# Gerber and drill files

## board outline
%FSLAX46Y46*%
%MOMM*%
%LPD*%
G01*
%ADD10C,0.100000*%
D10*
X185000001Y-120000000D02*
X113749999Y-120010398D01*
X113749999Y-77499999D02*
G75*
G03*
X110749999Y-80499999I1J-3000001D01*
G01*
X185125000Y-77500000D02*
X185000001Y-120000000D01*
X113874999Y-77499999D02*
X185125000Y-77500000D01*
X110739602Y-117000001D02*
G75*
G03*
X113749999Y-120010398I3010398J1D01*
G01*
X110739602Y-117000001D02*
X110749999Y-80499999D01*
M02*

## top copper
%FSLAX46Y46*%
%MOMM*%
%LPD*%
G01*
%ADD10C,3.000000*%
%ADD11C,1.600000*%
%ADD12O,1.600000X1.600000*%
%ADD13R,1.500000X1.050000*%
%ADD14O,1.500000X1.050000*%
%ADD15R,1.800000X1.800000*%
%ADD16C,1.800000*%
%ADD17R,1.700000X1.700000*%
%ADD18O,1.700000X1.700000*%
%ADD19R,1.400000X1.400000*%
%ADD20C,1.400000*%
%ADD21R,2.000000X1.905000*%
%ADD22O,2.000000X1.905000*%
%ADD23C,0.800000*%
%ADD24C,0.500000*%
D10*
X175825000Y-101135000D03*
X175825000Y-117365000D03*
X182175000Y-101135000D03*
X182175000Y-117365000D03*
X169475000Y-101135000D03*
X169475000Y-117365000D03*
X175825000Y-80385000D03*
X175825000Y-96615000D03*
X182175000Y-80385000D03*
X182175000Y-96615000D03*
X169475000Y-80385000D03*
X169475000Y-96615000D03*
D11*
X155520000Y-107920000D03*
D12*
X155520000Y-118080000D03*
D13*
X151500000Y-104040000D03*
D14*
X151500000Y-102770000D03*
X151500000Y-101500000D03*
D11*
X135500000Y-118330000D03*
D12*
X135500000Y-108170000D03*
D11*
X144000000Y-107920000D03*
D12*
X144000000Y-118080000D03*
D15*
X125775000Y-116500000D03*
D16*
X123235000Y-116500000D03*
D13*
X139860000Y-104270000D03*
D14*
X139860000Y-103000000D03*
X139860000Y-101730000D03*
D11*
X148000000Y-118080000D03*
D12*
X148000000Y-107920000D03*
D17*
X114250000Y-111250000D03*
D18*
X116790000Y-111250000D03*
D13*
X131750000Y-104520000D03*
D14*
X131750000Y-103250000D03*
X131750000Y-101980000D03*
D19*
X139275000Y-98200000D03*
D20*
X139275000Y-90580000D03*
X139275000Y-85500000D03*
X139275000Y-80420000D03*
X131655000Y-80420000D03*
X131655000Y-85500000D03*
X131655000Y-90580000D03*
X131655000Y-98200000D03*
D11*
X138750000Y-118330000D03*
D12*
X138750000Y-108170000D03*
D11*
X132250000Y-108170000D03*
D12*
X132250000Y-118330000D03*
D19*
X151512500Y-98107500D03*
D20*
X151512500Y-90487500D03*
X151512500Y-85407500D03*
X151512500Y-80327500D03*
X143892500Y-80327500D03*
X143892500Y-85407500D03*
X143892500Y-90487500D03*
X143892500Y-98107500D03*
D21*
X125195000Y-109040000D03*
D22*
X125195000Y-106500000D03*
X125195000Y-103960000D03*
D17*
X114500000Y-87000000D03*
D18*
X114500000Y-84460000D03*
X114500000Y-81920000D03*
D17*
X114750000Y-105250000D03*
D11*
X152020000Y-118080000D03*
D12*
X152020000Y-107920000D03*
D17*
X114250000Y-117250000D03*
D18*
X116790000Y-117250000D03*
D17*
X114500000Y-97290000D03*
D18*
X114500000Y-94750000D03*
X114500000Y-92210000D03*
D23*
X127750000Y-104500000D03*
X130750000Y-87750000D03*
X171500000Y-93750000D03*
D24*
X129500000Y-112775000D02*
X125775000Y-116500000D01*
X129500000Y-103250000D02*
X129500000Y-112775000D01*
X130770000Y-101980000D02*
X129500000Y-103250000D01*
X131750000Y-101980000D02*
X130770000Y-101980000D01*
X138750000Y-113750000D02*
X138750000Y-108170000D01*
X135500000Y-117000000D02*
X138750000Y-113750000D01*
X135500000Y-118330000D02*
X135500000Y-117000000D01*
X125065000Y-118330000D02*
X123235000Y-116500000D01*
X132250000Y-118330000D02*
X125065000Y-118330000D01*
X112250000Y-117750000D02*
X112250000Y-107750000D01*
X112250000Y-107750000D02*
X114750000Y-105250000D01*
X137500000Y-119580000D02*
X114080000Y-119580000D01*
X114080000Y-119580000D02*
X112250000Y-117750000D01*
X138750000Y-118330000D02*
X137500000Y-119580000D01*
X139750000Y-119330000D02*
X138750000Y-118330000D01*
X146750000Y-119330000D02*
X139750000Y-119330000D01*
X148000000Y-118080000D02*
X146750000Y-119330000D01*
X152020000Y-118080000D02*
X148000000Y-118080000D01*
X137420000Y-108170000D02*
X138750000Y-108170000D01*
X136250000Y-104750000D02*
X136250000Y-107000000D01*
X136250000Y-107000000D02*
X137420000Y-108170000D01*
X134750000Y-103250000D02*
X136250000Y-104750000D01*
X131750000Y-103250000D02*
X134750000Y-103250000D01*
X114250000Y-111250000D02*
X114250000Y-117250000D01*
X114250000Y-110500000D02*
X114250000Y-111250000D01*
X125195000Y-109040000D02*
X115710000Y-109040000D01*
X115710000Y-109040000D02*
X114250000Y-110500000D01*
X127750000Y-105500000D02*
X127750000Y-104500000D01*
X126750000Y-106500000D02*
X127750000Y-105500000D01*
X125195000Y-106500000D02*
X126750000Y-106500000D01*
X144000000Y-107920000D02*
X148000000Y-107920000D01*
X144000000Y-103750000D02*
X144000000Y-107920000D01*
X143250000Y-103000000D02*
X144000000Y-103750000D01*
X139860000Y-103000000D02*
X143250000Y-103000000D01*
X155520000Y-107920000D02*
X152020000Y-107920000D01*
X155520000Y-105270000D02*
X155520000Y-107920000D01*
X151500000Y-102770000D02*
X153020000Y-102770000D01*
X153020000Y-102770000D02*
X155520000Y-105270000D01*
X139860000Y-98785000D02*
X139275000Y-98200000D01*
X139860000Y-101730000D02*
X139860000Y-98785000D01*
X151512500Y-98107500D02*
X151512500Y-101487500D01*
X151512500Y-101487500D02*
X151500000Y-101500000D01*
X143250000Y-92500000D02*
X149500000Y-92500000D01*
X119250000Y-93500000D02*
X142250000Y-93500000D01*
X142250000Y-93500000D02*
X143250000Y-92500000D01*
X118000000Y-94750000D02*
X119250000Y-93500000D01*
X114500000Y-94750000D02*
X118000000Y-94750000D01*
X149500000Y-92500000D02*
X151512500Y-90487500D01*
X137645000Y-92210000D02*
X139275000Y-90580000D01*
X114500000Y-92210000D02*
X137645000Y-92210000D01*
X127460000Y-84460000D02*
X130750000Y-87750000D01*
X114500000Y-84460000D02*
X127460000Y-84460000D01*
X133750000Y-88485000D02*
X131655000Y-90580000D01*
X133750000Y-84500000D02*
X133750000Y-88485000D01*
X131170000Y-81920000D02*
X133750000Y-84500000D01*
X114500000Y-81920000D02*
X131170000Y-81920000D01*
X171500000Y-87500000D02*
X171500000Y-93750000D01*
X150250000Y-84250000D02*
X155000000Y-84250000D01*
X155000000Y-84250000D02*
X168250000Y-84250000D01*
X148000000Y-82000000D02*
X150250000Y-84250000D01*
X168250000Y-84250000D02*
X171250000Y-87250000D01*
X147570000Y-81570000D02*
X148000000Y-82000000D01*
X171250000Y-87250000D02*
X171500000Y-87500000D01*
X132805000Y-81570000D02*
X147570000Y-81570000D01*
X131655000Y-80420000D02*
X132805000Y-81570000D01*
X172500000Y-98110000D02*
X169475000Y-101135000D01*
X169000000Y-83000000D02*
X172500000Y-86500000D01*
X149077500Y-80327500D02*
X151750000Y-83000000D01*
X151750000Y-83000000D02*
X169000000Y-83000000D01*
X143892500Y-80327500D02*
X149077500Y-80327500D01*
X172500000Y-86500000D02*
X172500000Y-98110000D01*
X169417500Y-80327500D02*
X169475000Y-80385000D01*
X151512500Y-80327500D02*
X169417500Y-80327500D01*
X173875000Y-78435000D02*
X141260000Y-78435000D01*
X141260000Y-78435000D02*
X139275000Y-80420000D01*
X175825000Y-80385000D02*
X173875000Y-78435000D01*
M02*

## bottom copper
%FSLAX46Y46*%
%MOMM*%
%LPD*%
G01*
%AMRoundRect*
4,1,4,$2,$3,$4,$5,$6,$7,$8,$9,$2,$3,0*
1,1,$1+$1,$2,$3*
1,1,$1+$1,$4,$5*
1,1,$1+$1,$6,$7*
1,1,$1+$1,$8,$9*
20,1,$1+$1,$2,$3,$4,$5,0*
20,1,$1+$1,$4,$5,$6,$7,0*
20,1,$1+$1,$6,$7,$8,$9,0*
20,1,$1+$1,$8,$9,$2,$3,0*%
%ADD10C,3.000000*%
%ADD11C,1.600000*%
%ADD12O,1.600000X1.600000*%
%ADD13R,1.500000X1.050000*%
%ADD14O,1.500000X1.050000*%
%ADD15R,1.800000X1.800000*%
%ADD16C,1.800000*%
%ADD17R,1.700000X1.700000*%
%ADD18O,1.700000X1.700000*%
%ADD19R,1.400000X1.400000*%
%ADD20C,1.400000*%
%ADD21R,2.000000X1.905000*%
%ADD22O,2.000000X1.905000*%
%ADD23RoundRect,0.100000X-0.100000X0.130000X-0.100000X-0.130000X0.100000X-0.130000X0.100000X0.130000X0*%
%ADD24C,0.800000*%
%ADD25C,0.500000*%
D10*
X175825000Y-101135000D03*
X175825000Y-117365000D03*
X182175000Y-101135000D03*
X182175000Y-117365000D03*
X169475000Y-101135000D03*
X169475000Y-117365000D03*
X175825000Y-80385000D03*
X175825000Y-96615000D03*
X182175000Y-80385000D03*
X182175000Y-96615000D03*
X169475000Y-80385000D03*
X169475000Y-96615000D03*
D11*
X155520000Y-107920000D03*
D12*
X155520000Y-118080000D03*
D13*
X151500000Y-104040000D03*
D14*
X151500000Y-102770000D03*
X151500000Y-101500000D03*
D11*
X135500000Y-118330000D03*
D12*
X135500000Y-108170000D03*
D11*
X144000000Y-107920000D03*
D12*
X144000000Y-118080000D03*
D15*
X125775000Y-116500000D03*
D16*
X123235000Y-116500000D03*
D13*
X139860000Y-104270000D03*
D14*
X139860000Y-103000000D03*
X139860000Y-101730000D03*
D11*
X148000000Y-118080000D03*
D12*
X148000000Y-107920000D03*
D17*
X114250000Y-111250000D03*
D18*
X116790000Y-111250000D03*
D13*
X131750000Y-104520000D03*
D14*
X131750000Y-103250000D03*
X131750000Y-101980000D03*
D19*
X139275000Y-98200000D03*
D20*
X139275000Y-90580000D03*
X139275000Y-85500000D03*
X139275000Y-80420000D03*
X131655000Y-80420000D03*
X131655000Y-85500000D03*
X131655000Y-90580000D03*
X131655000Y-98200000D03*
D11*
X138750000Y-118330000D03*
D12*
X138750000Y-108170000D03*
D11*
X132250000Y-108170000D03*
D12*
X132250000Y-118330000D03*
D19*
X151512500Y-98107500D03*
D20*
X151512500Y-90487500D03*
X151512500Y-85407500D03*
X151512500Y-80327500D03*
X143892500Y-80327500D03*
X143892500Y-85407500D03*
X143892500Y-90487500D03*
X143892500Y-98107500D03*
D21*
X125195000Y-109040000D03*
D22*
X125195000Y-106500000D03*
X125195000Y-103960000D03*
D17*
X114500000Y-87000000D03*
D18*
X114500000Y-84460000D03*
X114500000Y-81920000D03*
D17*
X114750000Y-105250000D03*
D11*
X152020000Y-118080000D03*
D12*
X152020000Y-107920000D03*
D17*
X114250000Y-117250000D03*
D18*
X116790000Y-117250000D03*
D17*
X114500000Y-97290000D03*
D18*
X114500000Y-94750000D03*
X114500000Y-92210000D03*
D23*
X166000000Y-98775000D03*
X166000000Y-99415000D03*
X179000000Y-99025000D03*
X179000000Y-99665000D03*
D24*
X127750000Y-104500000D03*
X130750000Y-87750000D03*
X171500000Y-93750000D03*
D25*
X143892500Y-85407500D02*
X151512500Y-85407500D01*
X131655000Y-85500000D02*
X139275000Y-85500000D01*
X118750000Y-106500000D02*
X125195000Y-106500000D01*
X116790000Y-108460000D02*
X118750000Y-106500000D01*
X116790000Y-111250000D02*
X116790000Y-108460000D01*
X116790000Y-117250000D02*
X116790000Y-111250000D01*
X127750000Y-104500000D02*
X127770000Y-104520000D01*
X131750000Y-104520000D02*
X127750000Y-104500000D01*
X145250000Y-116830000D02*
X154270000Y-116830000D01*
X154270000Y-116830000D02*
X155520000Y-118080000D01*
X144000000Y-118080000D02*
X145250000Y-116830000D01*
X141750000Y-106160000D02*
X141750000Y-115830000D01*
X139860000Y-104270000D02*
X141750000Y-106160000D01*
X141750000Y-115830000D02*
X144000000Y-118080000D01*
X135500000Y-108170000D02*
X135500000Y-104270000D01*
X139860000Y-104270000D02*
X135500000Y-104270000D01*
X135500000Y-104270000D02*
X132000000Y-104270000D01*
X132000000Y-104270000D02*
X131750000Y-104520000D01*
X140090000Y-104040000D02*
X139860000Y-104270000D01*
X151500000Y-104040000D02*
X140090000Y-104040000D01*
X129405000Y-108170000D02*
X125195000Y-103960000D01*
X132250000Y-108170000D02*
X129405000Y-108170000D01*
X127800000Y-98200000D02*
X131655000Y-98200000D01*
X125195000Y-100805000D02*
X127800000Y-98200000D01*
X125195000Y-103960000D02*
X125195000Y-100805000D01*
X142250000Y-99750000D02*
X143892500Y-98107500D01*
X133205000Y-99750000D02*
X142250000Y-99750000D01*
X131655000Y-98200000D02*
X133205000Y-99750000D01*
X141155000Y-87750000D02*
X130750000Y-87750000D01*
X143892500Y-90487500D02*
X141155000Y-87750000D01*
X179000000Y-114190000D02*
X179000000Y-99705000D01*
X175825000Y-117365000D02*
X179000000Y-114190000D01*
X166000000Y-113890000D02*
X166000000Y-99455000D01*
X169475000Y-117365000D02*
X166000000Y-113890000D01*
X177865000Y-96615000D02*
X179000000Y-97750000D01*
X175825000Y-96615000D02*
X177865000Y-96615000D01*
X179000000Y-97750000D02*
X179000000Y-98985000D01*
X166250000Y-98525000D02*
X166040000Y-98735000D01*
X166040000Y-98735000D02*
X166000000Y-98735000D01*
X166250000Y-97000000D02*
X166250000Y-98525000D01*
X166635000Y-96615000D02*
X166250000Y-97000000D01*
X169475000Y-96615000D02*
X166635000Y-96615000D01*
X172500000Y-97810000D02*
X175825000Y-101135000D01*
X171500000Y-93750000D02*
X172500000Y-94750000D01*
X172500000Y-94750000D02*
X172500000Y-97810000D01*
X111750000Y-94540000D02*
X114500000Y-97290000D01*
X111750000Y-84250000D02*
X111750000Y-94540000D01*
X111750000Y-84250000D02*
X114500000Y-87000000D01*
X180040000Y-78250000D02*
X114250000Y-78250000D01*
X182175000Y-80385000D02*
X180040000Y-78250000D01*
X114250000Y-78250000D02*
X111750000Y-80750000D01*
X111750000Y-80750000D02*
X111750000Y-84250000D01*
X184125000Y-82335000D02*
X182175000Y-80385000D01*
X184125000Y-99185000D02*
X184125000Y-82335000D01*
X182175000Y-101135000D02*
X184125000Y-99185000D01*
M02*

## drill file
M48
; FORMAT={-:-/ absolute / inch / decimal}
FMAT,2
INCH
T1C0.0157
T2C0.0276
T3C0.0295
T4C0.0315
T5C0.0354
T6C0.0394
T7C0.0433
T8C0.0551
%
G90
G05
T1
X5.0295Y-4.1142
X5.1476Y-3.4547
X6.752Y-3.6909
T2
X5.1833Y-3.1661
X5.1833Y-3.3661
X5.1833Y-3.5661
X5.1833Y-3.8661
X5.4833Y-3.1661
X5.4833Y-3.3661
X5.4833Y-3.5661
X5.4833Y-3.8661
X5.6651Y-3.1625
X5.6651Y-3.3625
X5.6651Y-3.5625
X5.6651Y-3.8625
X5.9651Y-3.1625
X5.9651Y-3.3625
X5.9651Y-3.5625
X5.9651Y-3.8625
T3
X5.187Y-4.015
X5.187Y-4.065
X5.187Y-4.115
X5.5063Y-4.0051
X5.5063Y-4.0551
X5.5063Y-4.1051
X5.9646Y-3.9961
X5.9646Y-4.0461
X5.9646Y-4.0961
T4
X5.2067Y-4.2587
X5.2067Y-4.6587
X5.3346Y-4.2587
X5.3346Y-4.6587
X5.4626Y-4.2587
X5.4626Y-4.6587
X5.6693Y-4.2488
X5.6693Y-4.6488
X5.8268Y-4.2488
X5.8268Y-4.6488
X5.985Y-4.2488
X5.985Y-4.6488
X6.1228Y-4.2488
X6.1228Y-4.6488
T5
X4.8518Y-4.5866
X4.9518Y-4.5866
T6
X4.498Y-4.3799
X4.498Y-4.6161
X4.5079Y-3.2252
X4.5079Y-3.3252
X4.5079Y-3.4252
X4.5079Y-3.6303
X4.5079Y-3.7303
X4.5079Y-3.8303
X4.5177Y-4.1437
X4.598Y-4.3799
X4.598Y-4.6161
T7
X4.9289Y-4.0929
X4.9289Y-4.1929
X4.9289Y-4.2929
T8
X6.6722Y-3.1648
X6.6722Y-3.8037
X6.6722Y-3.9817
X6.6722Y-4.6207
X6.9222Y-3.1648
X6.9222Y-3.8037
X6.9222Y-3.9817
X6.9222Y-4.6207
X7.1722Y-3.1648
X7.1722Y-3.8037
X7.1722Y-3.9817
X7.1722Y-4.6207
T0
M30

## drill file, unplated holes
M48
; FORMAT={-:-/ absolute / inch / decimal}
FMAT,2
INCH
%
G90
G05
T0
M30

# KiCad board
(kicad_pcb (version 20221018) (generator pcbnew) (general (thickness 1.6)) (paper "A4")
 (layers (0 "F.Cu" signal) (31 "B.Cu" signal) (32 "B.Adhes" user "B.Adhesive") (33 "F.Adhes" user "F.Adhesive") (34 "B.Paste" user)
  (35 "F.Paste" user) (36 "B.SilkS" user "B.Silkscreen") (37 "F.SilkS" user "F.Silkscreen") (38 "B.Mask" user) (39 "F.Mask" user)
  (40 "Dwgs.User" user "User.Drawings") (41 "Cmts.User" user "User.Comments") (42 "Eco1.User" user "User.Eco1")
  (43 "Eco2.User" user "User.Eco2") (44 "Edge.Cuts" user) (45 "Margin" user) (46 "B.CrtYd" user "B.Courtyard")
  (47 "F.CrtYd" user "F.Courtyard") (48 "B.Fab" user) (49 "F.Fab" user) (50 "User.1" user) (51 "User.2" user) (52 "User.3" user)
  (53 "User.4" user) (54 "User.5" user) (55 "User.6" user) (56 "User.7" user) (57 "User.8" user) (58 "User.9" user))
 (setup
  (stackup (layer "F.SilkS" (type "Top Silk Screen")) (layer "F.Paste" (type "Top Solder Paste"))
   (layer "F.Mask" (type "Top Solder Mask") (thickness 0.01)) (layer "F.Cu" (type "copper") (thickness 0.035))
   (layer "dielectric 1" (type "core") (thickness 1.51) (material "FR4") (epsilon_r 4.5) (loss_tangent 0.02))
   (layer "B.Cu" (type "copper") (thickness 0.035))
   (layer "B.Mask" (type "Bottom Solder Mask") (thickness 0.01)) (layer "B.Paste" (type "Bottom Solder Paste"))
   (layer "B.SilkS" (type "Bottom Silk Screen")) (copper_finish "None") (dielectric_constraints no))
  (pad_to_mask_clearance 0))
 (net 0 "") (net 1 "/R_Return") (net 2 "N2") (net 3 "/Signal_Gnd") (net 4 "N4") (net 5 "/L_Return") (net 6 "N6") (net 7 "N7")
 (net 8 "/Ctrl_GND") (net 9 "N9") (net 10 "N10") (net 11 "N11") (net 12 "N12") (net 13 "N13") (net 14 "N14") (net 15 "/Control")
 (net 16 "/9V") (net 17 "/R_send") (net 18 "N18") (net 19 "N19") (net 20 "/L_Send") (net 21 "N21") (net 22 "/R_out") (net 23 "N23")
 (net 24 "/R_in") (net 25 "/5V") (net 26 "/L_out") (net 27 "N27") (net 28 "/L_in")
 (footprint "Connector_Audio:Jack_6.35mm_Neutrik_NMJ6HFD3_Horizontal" (layer "F.Cu") (at 169.475 80.385)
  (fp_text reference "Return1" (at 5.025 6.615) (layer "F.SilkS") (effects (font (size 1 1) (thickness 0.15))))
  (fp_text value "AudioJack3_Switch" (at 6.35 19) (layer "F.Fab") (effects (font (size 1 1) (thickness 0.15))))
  (pad "R" thru_hole circle (at 6.35 0) (size 3 3) (drill 1.4) (layers "*.Cu" "*.Mask") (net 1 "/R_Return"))
  (pad "RN" thru_hole circle (at 6.35 16.23) (size 3 3) (drill 1.4) (layers "*.Cu" "*.Mask") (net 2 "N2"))
  (pad "S" thru_hole circle (at 12.7 0) (size 3 3) (drill 1.4) (layers "*.Cu" "*.Mask") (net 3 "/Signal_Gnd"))
  (pad "SN" thru_hole circle (at 12.7 16.23) (size 3 3) (drill 1.4) (layers "*.Cu" "*.Mask") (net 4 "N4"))
  (pad "T" thru_hole circle (at 0 0) (size 3 3) (drill 1.4) (layers "*.Cu" "*.Mask") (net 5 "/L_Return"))
  (pad "TN" thru_hole circle (at 0 16.23) (size 3 3) (drill 1.4) (layers "*.Cu" "*.Mask") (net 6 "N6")))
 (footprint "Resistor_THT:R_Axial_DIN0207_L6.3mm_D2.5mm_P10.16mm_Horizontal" (layer "F.Cu") (at 155.52 107.92 -90)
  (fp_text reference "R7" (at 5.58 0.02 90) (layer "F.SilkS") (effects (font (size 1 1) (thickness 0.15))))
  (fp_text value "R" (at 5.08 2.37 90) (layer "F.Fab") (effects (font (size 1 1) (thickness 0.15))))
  (pad "1" thru_hole circle (at 0 0 270) (size 1.6 1.6) (drill 0.8) (layers "*.Cu" "*.Mask") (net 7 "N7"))
  (pad "2" thru_hole oval (at 10.16 0 270) (size 1.6 1.6) (drill 0.8) (layers "*.Cu" "*.Mask") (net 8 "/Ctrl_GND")))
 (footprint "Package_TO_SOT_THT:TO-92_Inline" (layer "F.Cu") (at 151.5 104.04 90)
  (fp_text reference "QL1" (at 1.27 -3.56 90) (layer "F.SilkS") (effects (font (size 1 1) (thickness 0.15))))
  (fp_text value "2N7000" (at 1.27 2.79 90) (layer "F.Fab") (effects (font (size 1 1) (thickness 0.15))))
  (pad "1" thru_hole rect (at 0 0 90) (size 1.05 1.5) (drill 0.75) (layers "*.Cu" "*.Mask") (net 8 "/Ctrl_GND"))
  (pad "2" thru_hole oval (at 1.27 0 90) (size 1.05 1.5) (drill 0.75) (layers "*.Cu" "*.Mask") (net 7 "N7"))
  (pad "3" thru_hole oval (at 2.54 0 90) (size 1.05 1.5) (drill 0.75) (layers "*.Cu" "*.Mask") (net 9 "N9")))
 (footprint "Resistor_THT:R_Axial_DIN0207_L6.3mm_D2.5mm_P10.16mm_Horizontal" (layer "F.Cu") (at 135.5 118.33 90)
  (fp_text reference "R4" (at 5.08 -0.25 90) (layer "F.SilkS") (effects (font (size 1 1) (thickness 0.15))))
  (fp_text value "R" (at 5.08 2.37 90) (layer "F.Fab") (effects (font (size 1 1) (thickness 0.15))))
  (pad "1" thru_hole circle (at 0 0 90) (size 1.6 1.6) (drill 0.8) (layers "*.Cu" "*.Mask") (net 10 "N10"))
  (pad "2" thru_hole oval (at 10.16 0 90) (size 1.6 1.6) (drill 0.8) (layers "*.Cu" "*.Mask") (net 8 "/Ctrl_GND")))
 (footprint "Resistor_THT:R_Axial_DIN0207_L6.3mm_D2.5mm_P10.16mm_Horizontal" (layer "F.Cu") (at 144 107.92 -90)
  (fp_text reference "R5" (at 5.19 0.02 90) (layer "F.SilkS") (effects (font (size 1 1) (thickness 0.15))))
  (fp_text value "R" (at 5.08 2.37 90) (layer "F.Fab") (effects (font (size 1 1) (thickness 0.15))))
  (pad "1" thru_hole circle (at 0 0 270) (size 1.6 1.6) (drill 0.8) (layers "*.Cu" "*.Mask") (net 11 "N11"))
  (pad "2" thru_hole oval (at 10.16 0 270) (size 1.6 1.6) (drill 0.8) (layers "*.Cu" "*.Mask") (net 8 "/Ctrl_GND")))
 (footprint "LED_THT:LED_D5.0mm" (layer "F.Cu") (at 125.775 116.5 180)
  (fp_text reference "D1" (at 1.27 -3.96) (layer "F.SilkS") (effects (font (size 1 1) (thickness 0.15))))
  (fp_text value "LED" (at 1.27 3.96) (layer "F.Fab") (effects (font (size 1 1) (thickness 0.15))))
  (pad "1" thru_hole rect (at 0 0 180) (size 1.8 1.8) (drill 0.9) (layers "*.Cu" "*.Mask") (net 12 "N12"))
  (pad "2" thru_hole circle (at 2.54 0 180) (size 1.8 1.8) (drill 0.9) (layers "*.Cu" "*.Mask") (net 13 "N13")))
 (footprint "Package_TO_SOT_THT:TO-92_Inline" (layer "F.Cu") (at 139.86 104.27 90)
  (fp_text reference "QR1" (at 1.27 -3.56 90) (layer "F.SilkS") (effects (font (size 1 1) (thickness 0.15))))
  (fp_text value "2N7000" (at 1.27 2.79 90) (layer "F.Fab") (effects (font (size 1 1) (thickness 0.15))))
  (pad "1" thru_hole rect (at 0 0 90) (size 1.05 1.5) (drill 0.75) (layers "*.Cu" "*.Mask") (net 8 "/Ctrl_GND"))
  (pad "2" thru_hole oval (at 1.27 0 90) (size 1.05 1.5) (drill 0.75) (layers "*.Cu" "*.Mask") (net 11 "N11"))
  (pad "3" thru_hole oval (at 2.54 0 90) (size 1.05 1.5) (drill 0.75) (layers "*.Cu" "*.Mask") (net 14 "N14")))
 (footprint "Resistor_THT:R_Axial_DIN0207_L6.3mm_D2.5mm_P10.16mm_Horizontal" (layer "F.Cu") (at 148 118.08 90)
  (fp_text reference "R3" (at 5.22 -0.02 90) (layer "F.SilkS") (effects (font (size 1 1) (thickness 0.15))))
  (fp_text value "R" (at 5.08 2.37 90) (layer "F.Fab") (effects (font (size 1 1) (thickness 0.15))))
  (pad "1" thru_hole circle (at 0 0 90) (size 1.6 1.6) (drill 0.8) (layers "*.Cu" "*.Mask") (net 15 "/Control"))
  (pad "2" thru_hole oval (at 10.16 0 90) (size 1.6 1.6) (drill 0.8) (layers "*.Cu" "*.Mask") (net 11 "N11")))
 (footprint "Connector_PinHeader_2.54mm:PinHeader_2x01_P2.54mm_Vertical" (layer "F.Cu") (at 114.25 111.25)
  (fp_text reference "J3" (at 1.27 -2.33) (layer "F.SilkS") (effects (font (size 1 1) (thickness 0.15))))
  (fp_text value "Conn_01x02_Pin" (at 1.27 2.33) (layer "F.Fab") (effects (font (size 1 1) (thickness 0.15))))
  (pad "1" thru_hole rect (at 0 0) (size 1.7 1.7) (drill 1) (layers "*.Cu" "*.Mask") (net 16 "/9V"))
  (pad "2" thru_hole oval (at 2.54 0) (size 1.7 1.7) (drill 1) (layers "*.Cu" "*.Mask") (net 8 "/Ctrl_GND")))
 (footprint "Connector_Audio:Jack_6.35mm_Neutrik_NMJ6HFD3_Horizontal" (layer "F.Cu") (at 169.475 101.135)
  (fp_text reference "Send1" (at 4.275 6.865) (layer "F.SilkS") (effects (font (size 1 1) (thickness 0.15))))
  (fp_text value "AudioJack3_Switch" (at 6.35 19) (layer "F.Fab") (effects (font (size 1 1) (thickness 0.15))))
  (pad "R" thru_hole circle (at 6.35 0) (size 3 3) (drill 1.4) (layers "*.Cu" "*.Mask") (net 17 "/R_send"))
  (pad "RN" thru_hole circle (at 6.35 16.23) (size 3 3) (drill 1.4) (layers "*.Cu" "*.Mask") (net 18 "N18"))
  (pad "S" thru_hole circle (at 12.7 0) (size 3 3) (drill 1.4) (layers "*.Cu" "*.Mask") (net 3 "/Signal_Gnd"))
  (pad "SN" thru_hole circle (at 12.7 16.23) (size 3 3) (drill 1.4) (layers "*.Cu" "*.Mask") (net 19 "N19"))
  (pad "T" thru_hole circle (at 0 0) (size 3 3) (drill 1.4) (layers "*.Cu" "*.Mask") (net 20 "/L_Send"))
  (pad "TN" thru_hole circle (at 0 16.23) (size 3 3) (drill 1.4) (layers "*.Cu" "*.Mask") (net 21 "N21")))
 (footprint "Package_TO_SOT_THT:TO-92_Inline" (layer "F.Cu") (at 131.75 104.52 90)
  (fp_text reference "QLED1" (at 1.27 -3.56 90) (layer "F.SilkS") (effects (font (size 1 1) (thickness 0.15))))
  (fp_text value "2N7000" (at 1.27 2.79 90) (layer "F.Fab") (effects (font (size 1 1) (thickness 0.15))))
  (pad "1" thru_hole rect (at 0 0 90) (size 1.05 1.5) (drill 0.75) (layers "*.Cu" "*.Mask") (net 8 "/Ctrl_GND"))
  (pad "2" thru_hole oval (at 1.27 0 90) (size 1.05 1.5) (drill 0.75) (layers "*.Cu" "*.Mask") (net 10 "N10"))
  (pad "3" thru_hole oval (at 2.54 0 90) (size 1.05 1.5) (drill 0.75) (layers "*.Cu" "*.Mask") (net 12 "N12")))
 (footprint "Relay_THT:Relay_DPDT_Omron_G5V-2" (layer "F.Cu") (at 139.275 98.2 180)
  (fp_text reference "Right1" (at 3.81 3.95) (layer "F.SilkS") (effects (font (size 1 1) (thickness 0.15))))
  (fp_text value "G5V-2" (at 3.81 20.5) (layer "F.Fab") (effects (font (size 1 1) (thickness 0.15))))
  (pad "1" thru_hole rect (at 0 0 180) (size 1.4 1.4) (drill 0.7) (layers "*.Cu" "*.Mask") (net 14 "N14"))
  (pad "4" thru_hole circle (at 0 7.62 180) (size 1.4 1.4) (drill 0.7) (layers "*.Cu" "*.Mask") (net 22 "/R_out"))
  (pad "6" thru_hole circle (at 0 12.7 180) (size 1.4 1.4) (drill 0.7) (layers "*.Cu" "*.Mask") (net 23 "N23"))
  (pad "8" thru_hole circle (at 0 17.78 180) (size 1.4 1.4) (drill 0.7) (layers "*.Cu" "*.Mask") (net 1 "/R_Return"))
  (pad "9" thru_hole circle (at 7.62 17.78 180) (size 1.4 1.4) (drill 0.7) (layers "*.Cu" "*.Mask") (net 17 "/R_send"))
  (pad "11" thru_hole circle (at 7.62 12.7 180) (size 1.4 1.4) (drill 0.7) (layers "*.Cu" "*.Mask") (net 23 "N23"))
  (pad "13" thru_hole circle (at 7.62 7.62 180) (size 1.4 1.4) (drill 0.7) (layers "*.Cu" "*.Mask") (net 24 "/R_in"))
  (pad "16" thru_hole circle (at 7.62 0 180) (size 1.4 1.4) (drill 0.7) (layers "*.Cu" "*.Mask") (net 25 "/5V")))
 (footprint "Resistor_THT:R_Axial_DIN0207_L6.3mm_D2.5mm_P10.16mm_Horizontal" (layer "F.Cu") (at 138.75 118.33 90)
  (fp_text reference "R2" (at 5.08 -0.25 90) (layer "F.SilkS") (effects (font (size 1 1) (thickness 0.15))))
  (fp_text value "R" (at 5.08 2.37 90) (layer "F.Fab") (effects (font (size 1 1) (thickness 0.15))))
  (pad "1" thru_hole circle (at 0 0 90) (size 1.6 1.6) (drill 0.8) (layers "*.Cu" "*.Mask") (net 15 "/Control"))
  (pad "2" thru_hole oval (at 10.16 0 90) (size 1.6 1.6) (drill 0.8) (layers "*.Cu" "*.Mask") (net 10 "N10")))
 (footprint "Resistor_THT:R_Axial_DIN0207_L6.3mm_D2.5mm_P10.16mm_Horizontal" (layer "F.Cu") (at 132.25 108.17 -90)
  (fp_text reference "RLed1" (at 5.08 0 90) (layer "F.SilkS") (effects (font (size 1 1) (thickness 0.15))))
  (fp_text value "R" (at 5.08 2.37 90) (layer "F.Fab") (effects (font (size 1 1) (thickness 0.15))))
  (pad "1" thru_hole circle (at 0 0 270) (size 1.6 1.6) (drill 0.8) (layers "*.Cu" "*.Mask") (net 25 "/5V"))
  (pad "2" thru_hole oval (at 10.16 0 270) (size 1.6 1.6) (drill 0.8) (layers "*.Cu" "*.Mask") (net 13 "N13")))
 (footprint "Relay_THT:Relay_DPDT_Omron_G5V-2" (layer "F.Cu") (at 151.5125 98.1075 180)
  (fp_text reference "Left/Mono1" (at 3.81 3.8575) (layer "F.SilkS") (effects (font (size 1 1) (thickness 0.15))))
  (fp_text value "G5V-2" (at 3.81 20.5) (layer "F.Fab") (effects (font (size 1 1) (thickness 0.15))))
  (pad "1" thru_hole rect (at 0 0 180) (size 1.4 1.4) (drill 0.7) (layers "*.Cu" "*.Mask") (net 9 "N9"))
  (pad "4" thru_hole circle (at 0 7.62 180) (size 1.4 1.4) (drill 0.7) (layers "*.Cu" "*.Mask") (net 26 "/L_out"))
  (pad "6" thru_hole circle (at 0 12.7 180) (size 1.4 1.4) (drill 0.7) (layers "*.Cu" "*.Mask") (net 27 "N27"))
  (pad "8" thru_hole circle (at 0 17.78 180) (size 1.4 1.4) (drill 0.7) (layers "*.Cu" "*.Mask") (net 5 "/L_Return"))
  (pad "9" thru_hole circle (at 7.62 17.78 180) (size 1.4 1.4) (drill 0.7) (layers "*.Cu" "*.Mask") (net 20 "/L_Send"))
  (pad "11" thru_hole circle (at 7.62 12.7 180) (size 1.4 1.4) (drill 0.7) (layers "*.Cu" "*.Mask") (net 27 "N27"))
  (pad "13" thru_hole circle (at 7.62 7.62 180) (size 1.4 1.4) (drill 0.7) (layers "*.Cu" "*.Mask") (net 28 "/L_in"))
  (pad "16" thru_hole circle (at 7.62 0 180) (size 1.4 1.4) (drill 0.7) (layers "*.Cu" "*.Mask") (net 25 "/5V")))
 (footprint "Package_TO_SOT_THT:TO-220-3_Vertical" (layer "F.Cu") (at 125.195 109.04 90)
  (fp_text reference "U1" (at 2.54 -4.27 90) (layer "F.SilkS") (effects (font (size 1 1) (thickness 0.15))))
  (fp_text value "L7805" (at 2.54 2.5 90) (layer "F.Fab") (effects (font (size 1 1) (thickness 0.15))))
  (pad "1" thru_hole rect (at 0 0 90) (size 1.905 2) (drill 1.1) (layers "*.Cu" "*.Mask") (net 16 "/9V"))
  (pad "2" thru_hole oval (at 2.54 0 90) (size 1.905 2) (drill 1.1) (layers "*.Cu" "*.Mask") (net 8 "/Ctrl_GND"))
  (pad "3" thru_hole oval (at 5.08 0 90) (size 1.905 2) (drill 1.1) (layers "*.Cu" "*.Mask") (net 25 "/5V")))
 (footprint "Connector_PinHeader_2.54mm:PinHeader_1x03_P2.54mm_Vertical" (layer "F.Cu") (at 114.5 87 180)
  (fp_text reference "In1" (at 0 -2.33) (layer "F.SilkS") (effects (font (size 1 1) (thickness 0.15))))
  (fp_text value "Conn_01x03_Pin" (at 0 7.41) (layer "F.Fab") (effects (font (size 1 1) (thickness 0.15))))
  (pad "1" thru_hole rect (at 0 0 180) (size 1.7 1.7) (drill 1) (layers "*.Cu" "*.Mask") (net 3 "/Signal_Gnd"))
  (pad "2" thru_hole oval (at 0 2.54 180) (size 1.7 1.7) (drill 1) (layers "*.Cu" "*.Mask") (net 28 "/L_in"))
  (pad "3" thru_hole oval (at 0 5.08 180) (size 1.7 1.7) (drill 1) (layers "*.Cu" "*.Mask") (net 24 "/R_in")))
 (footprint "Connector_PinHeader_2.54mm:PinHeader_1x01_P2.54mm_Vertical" (layer "F.Cu") (at 114.75 105.25)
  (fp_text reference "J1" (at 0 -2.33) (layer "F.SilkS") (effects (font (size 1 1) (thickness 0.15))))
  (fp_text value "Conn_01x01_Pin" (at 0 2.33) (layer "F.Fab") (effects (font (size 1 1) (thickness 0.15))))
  (pad "1" thru_hole rect (at 0 0) (size 1.7 1.7) (drill 1) (layers "*.Cu" "*.Mask") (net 15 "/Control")))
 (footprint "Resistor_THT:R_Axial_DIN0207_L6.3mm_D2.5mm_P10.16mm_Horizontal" (layer "F.Cu") (at 152.02 118.08 90)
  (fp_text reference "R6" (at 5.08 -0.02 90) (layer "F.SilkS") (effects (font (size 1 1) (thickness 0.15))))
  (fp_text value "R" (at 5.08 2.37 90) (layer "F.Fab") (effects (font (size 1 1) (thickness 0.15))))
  (pad "1" thru_hole circle (at 0 0 90) (size 1.6 1.6) (drill 0.8) (layers "*.Cu" "*.Mask") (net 15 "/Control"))
  (pad "2" thru_hole oval (at 10.16 0 90) (size 1.6 1.6) (drill 0.8) (layers "*.Cu" "*.Mask") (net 7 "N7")))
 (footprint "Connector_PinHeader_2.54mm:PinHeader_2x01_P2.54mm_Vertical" (layer "F.Cu") (at 114.25 117.25)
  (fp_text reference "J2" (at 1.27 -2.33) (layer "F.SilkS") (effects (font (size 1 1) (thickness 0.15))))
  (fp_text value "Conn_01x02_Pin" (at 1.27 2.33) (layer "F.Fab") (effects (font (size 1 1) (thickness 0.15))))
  (pad "1" thru_hole rect (at 0 0) (size 1.7 1.7) (drill 1) (layers "*.Cu" "*.Mask") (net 16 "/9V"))
  (pad "2" thru_hole oval (at 2.54 0) (size 1.7 1.7) (drill 1) (layers "*.Cu" "*.Mask") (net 8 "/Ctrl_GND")))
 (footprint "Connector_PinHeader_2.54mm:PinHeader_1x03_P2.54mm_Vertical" (layer "F.Cu") (at 114.5 97.29 180)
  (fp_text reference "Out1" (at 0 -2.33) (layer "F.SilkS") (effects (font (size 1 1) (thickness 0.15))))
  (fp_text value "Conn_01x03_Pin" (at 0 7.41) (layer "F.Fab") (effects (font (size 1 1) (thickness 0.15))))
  (pad "1" thru_hole rect (at 0 0 180) (size 1.7 1.7) (drill 1) (layers "*.Cu" "*.Mask") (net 3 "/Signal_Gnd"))
  (pad "2" thru_hole oval (at 0 2.54 180) (size 1.7 1.7) (drill 1) (layers "*.Cu" "*.Mask") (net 26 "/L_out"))
  (pad "3" thru_hole oval (at 0 5.08 180) (size 1.7 1.7) (drill 1) (layers "*.Cu" "*.Mask") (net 22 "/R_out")))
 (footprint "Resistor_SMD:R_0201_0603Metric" (layer "B.Cu") (at 166 99.095 -90)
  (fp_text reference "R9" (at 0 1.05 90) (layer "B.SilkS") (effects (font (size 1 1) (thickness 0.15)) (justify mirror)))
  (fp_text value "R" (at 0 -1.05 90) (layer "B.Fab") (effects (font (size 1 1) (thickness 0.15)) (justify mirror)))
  (pad "" smd roundrect (at -0.345 0 270) (size 0.318 0.36) (layers "B.Paste") (roundrect_rratio 0.25))
  (pad "" smd roundrect (at 0.345 0 270) (size 0.318 0.36) (layers "B.Paste") (roundrect_rratio 0.25))
  (pad "1" smd roundrect (at -0.32 0 270) (size 0.46 0.4) (layers "B.Cu" "B.Mask") (roundrect_rratio 0.25) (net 6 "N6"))
  (pad "2" smd roundrect (at 0.32 0 270) (size 0.46 0.4) (layers "B.Cu" "B.Mask") (roundrect_rratio 0.25) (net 21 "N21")))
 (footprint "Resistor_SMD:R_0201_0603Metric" (layer "B.Cu") (at 179 99.345 -90)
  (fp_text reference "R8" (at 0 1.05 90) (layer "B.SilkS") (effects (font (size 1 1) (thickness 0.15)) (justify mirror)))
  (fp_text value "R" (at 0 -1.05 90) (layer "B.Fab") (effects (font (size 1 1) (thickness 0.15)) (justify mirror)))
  (pad "" smd roundrect (at -0.345 0 270) (size 0.318 0.36) (layers "B.Paste") (roundrect_rratio 0.25))
  (pad "" smd roundrect (at 0.345 0 270) (size 0.318 0.36) (layers "B.Paste") (roundrect_rratio 0.25))
  (pad "1" smd roundrect (at -0.32 0 270) (size 0.46 0.4) (layers "B.Cu" "B.Mask") (roundrect_rratio 0.25) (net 2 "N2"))
  (pad "2" smd roundrect (at 0.32 0 270) (size 0.46 0.4) (layers "B.Cu" "B.Mask") (roundrect_rratio 0.25) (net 18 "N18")))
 (gr_line (start 185.000001 120) (end 113.749999 120.010398) (stroke (width 0.1) (type default)) (layer "Edge.Cuts"))
 (gr_arc (start 110.749999 80.499999) (mid 111.628679 78.378679) (end 113.749999 77.499999) (stroke (width 0.1) (type default))
  (layer "Edge.Cuts"))
 (gr_line (start 185.125 77.5) (end 185.000001 120) (stroke (width 0.1) (type default)) (layer "Edge.Cuts"))
 (gr_line (start 113.874999 77.499999) (end 185.125 77.5) (stroke (width 0.1) (type default)) (layer "Edge.Cuts"))
 (gr_arc (start 113.749999 120.010398) (mid 111.621327 119.128673) (end 110.739602 117.000001) (stroke (width 0.1) (type default))
  (layer "Edge.Cuts"))
 (gr_line (start 110.739602 117.000001) (end 110.749999 80.499999) (stroke (width 0.1) (type default)) (layer "Edge.Cuts"))
 (segment (start 139.75 119.33) (end 138.75 118.33) (width 0.5) (layer "F.Cu") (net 15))
 (segment (start 148 118.08) (end 146.75 119.33) (width 0.5) (layer "F.Cu") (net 15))
 (segment (start 152.02 118.08) (end 148 118.08) (width 0.5) (layer "F.Cu") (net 15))
 (segment (start 114.08 119.58) (end 112.25 117.75) (width 0.5) (layer "F.Cu") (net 15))
 (segment (start 146.75 119.33) (end 139.75 119.33) (width 0.5) (layer "F.Cu") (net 15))
 (segment (start 138.75 118.33) (end 137.5 119.58) (width 0.5) (layer "F.Cu") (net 15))
 (segment (start 137.5 119.58) (end 114.08 119.58) (width 0.5) (layer "F.Cu") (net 15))
 (segment (start 112.25 117.75) (end 112.25 107.75) (width 0.5) (layer "F.Cu") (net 15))
 (segment (start 112.25 107.75) (end 114.75 105.25) (width 0.5) (layer "F.Cu") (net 15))
 (segment (start 125.195 109.04) (end 115.71 109.04) (width 0.5) (layer "F.Cu") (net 16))
 (segment (start 115.71 109.04) (end 114.25 110.5) (width 0.5) (layer "F.Cu") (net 16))
 (segment (start 114.25 110.5) (end 114.25 111.25) (width 0.5) (layer "F.Cu") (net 16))
 (segment (start 114.25 111.25) (end 114.25 117.25) (width 0.5) (layer "F.Cu") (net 16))
 (segment (start 127.75 105.5) (end 127.75 104.5) (width 0.5) (layer "F.Cu") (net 8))
 (segment (start 126.75 106.5) (end 127.75 105.5) (width 0.5) (layer "F.Cu") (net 8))
 (segment (start 125.195 106.5) (end 126.75 106.5) (width 0.5) (layer "F.Cu") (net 8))
 (via (at 127.75 104.5) (size 0.8) (drill 0.4) (layers "F.Cu" "B.Cu") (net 8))
 (segment (start 141.75 106.16) (end 141.75 115.83) (width 0.5) (layer "B.Cu") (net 8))
 (segment (start 131.75 104.52) (end 127.75 104.5) (width 0.5) (layer "B.Cu") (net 8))
 (segment (start 118.75 106.5) (end 125.195 106.5) (width 0.5) (layer "B.Cu") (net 8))
 (segment (start 127.75 104.5) (end 127.77 104.52) (width 0.5) (layer "B.Cu") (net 8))
 (segment (start 116.79 108.46) (end 118.75 106.5) (width 0.5) (layer "B.Cu") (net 8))
 (segment (start 116.79 111.25) (end 116.79 108.46) (width 0.5) (layer "B.Cu") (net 8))
 (segment (start 116.79 117.25) (end 116.79 111.25) (width 0.5) (layer "B.Cu") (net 8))
 (segment (start 154.27 116.83) (end 155.52 118.08) (width 0.5) (layer "B.Cu") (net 8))
 (segment (start 139.86 104.27) (end 135.5 104.27) (width 0.5) (layer "B.Cu") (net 8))
 (segment (start 151.5 104.04) (end 140.09 104.04) (width 0.5) (layer "B.Cu") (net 8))
 (segment (start 132 104.27) (end 131.75 104.52) (width 0.5) (layer "B.Cu") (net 8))
 (segment (start 140.09 104.04) (end 139.86 104.27) (width 0.5) (layer "B.Cu") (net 8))
 (segment (start 141.75 115.83) (end 144 118.08) (width 0.5) (layer "B.Cu") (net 8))
 (segment (start 144 118.08) (end 145.25 116.83) (width 0.5) (layer "B.Cu") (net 8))
 (segment (start 145.25 116.83) (end 154.27 116.83) (width 0.5) (layer "B.Cu") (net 8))
 (segment (start 135.5 104.27) (end 132 104.27) (width 0.5) (layer "B.Cu") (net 8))
 (segment (start 139.86 104.27) (end 141.75 106.16) (width 0.5) (layer "B.Cu") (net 8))
 (segment (start 135.5 108.17) (end 135.5 104.27) (width 0.5) (layer "B.Cu") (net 8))
 (segment (start 131.75 101.98) (end 130.77 101.98) (width 0.5) (layer "F.Cu") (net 12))
 (segment (start 129.5 112.775) (end 125.775 116.5) (width 0.5) (layer "F.Cu") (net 12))
 (segment (start 129.5 103.25) (end 129.5 112.775) (width 0.5) (layer "F.Cu") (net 12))
 (segment (start 130.77 101.98) (end 129.5 103.25) (width 0.5) (layer "F.Cu") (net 12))
 (segment (start 125.065 118.33) (end 123.235 116.5) (width 0.5) (layer "F.Cu") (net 13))
 (segment (start 132.25 118.33) (end 125.065 118.33) (width 0.5) (layer "F.Cu") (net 13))
 (segment (start 131.17 81.92) (end 133.75 84.5) (width 0.5) (layer "F.Cu") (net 24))
 (segment (start 133.75 88.485) (end 131.655 90.58) (width 0.5) (layer "F.Cu") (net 24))
 (segment (start 114.5 81.92) (end 131.17 81.92) (width 0.5) (layer "F.Cu") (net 24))
 (segment (start 133.75 84.5) (end 133.75 88.485) (width 0.5) (layer "F.Cu") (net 24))
 (segment (start 127.46 84.46) (end 130.75 87.75) (width 0.5) (layer "F.Cu") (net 28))
 (segment (start 114.5 84.46) (end 127.46 84.46) (width 0.5) (layer "F.Cu") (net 28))
 (via (at 130.75 87.75) (size 0.8) (drill 0.4) (layers "F.Cu" "B.Cu") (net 28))
 (segment (start 143.8925 90.4875) (end 141.155 87.75) (width 0.5) (layer "B.Cu") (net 28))
 (segment (start 141.155 87.75) (end 130.75 87.75) (width 0.5) (layer "B.Cu") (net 28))
 (segment (start 182.175 101.135) (end 184.125 99.185) (width 0.5) (layer "B.Cu") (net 3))
 (segment (start 114.25 78.25) (end 111.75 80.75) (width 0.5) (layer "B.Cu") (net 3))
 (segment (start 111.75 84.25) (end 111.75 94.54) (width 0.5) (layer "B.Cu") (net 3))
 (segment (start 180.04 78.25) (end 114.25 78.25) (width 0.5) (layer "B.Cu") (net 3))
 (segment (start 184.125 99.185) (end 184.125 82.335) (width 0.5) (layer "B.Cu") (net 3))
 (segment (start 111.75 94.54) (end 114.5 97.29) (width 0.5) (layer "B.Cu") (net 3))
 (segment (start 111.75 84.25) (end 114.5 87) (width 0.5) (layer "B.Cu") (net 3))
 (segment (start 182.175 80.385) (end 180.04 78.25) (width 0.5) (layer "B.Cu") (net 3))
 (segment (start 184.125 82.335) (end 182.175 80.385) (width 0.5) (layer "B.Cu") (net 3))
 (segment (start 111.75 80.75) (end 111.75 84.25) (width 0.5) (layer "B.Cu") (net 3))
 (segment (start 137.645 92.21) (end 139.275 90.58) (width 0.5) (layer "F.Cu") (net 22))
 (segment (start 114.5 92.21) (end 137.645 92.21) (width 0.5) (layer "F.Cu") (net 22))
 (segment (start 175.825 80.385) (end 173.875 78.435) (width 0.5) (layer "F.Cu") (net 1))
 (segment (start 173.875 78.435) (end 141.26 78.435) (width 0.5) (layer "F.Cu") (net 1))
 (segment (start 141.26 78.435) (end 139.275 80.42) (width 0.5) (layer "F.Cu") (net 1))
 (segment (start 132.805 81.57) (end 147.57 81.57) (width 0.5) (layer "F.Cu") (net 17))
 (segment (start 171.5 87.5) (end 171.5 93.75) (width 0.5) (layer "F.Cu") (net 17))
 (segment (start 155 84.25) (end 168.25 84.25) (width 0.5) (layer "F.Cu") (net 17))
 (segment (start 150.25 84.25) (end 155 84.25) (width 0.5) (layer "F.Cu") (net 17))
 (segment (start 171.25 87.25) (end 171.5 87.5) (width 0.5) (layer "F.Cu") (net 17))
 (segment (start 147.57 81.57) (end 148 82) (width 0.5) (layer "F.Cu") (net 17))
 (segment (start 131.655 80.42) (end 132.805 81.57) (width 0.5) (layer "F.Cu") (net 17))
 (segment (start 148 82) (end 150.25 84.25) (width 0.5) (layer "F.Cu") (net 17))
 (segment (start 168.25 84.25) (end 171.25 87.25) (width 0.5) (layer "F.Cu") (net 17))
 (via (at 171.5 93.75) (size 0.8) (drill 0.4) (layers "F.Cu" "B.Cu") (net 17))
 (segment (start 172.5 94.75) (end 172.5 97.81) (width 0.5) (layer "B.Cu") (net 17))
 (segment (start 172.5 97.81) (end 175.825 101.135) (width 0.5) (layer "B.Cu") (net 17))
 (segment (start 171.5 93.75) (end 172.5 94.75) (width 0.5) (layer "B.Cu") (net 17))
 (segment (start 131.655 98.2) (end 133.205 99.75) (width 0.5) (layer "B.Cu") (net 25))
 (segment (start 142.25 99.75) (end 143.8925 98.1075) (width 0.5) (layer "B.Cu") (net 25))
 (segment (start 132.25 108.17) (end 129.405 108.17) (width 0.5) (layer "B.Cu") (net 25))
 (segment (start 125.195 100.805) (end 127.8 98.2) (width 0.5) (layer "B.Cu") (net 25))
 (segment (start 127.8 98.2) (end 131.655 98.2) (width 0.5) (layer "B.Cu") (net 25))
 (segment (start 125.195 103.96) (end 125.195 100.805) (width 0.5) (layer "B.Cu") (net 25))
 (segment (start 133.205 99.75) (end 142.25 99.75) (width 0.5) (layer "B.Cu") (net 25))
 (segment (start 129.405 108.17) (end 125.195 103.96) (width 0.5) (layer "B.Cu") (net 25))
 (segment (start 143.25 92.5) (end 149.5 92.5) (width 0.5) (layer "F.Cu") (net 26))
 (segment (start 119.25 93.5) (end 142.25 93.5) (width 0.5) (layer "F.Cu") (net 26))
 (segment (start 149.5 92.5) (end 151.5125 90.4875) (width 0.5) (layer "F.Cu") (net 26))
 (segment (start 142.25 93.5) (end 143.25 92.5) (width 0.5) (layer "F.Cu") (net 26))
 (segment (start 114.5 94.75) (end 118 94.75) (width 0.5) (layer "F.Cu") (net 26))
 (segment (start 118 94.75) (end 119.25 93.5) (width 0.5) (layer "F.Cu") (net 26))
 (segment (start 151.5125 80.3275) (end 169.4175 80.3275) (width 0.5) (layer "F.Cu") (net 5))
 (segment (start 169.4175 80.3275) (end 169.475 80.385) (width 0.5) (layer "F.Cu") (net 5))
 (segment (start 143.8925 80.3275) (end 149.0775 80.3275) (width 0.5) (layer "F.Cu") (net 20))
 (segment (start 149.0775 80.3275) (end 151.75 83) (width 0.5) (layer "F.Cu") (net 20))
 (segment (start 151.75 83) (end 169 83) (width 0.5) (layer "F.Cu") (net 20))
 (segment (start 172.5 98.11) (end 169.475 101.135) (width 0.5) (layer "F.Cu") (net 20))
 (segment (start 169 83) (end 172.5 86.5) (width 0.5) (layer "F.Cu") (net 20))
 (segment (start 172.5 86.5) (end 172.5 98.11) (width 0.5) (layer "F.Cu") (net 20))
 (segment (start 177.865 96.615) (end 179 97.75) (width 0.5) (layer "B.Cu") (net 2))
 (segment (start 179 97.75) (end 179 98.985) (width 0.5) (layer "B.Cu") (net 2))
 (segment (start 175.825 96.615) (end 177.865 96.615) (width 0.5) (layer "B.Cu") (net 2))
 (segment (start 175.825 117.365) (end 179 114.19) (width 0.5) (layer "B.Cu") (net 18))
 (segment (start 179 114.19) (end 179 99.705) (width 0.5) (layer "B.Cu") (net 18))
 (segment (start 169.475 96.615) (end 166.635 96.615) (width 0.5) (layer "B.Cu") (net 6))
 (segment (start 166.25 98.525) (end 166.04 98.735) (width 0.5) (layer "B.Cu") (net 6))
 (segment (start 166.04 98.735) (end 166 98.735) (width 0.5) (layer "B.Cu") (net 6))
 (segment (start 166.25 97) (end 166.25 98.525) (width 0.5) (layer "B.Cu") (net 6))
 (segment (start 166.635 96.615) (end 166.25 97) (width 0.5) (layer "B.Cu") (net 6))
 (segment (start 166 113.89) (end 166 99.455) (width 0.5) (layer "B.Cu") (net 21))
 (segment (start 169.475 117.365) (end 166 113.89) (width 0.5) (layer "B.Cu") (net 21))
 (segment (start 143.8925 85.4075) (end 151.5125 85.4075) (width 0.5) (layer "B.Cu") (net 27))
 (segment (start 131.655 85.5) (end 139.275 85.5) (width 0.5) (layer "B.Cu") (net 23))
 (segment (start 151.5125 98.1075) (end 151.5125 101.4875) (width 0.5) (layer "F.Cu") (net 9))
 (segment (start 151.5125 101.4875) (end 151.5 101.5) (width 0.5) (layer "F.Cu") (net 9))
 (segment (start 151.5 102.77) (end 153.02 102.77) (width 0.5) (layer "F.Cu") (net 7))
 (segment (start 153.02 102.77) (end 155.52 105.27) (width 0.5) (layer "F.Cu") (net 7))
 (segment (start 155.52 105.27) (end 155.52 107.92) (width 0.5) (layer "F.Cu") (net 7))
 (segment (start 155.52 107.92) (end 152.02 107.92) (width 0.5) (layer "F.Cu") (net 7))
 (segment (start 136.25 104.75) (end 136.25 107) (width 0.5) (layer "F.Cu") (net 10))
 (segment (start 136.25 107) (end 137.42 108.17) (width 0.5) (layer "F.Cu") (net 10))
 (segment (start 131.75 103.25) (end 134.75 103.25) (width 0.5) (layer "F.Cu") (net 10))
 (segment (start 138.75 113.75) (end 138.75 108.17) (width 0.5) (layer "F.Cu") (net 10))
 (segment (start 135.5 117) (end 138.75 113.75) (width 0.5) (layer "F.Cu") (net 10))
 (segment (start 137.42 108.17) (end 138.75 108.17) (width 0.5) (layer "F.Cu") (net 10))
 (segment (start 134.75 103.25) (end 136.25 104.75) (width 0.5) (layer "F.Cu") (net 10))
 (segment (start 135.5 118.33) (end 135.5 117) (width 0.5) (layer "F.Cu") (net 10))
 (segment (start 144 107.92) (end 148 107.92) (width 0.5) (layer "F.Cu") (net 11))
 (segment (start 144 103.75) (end 144 107.92) (width 0.5) (layer "F.Cu") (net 11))
 (segment (start 143.25 103) (end 144 103.75) (width 0.5) (layer "F.Cu") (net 11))
 (segment (start 139.86 103) (end 143.25 103) (width 0.5) (layer "F.Cu") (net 11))
 (segment (start 139.86 101.73) (end 139.86 98.785) (width 0.5) (layer "F.Cu") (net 14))
 (segment (start 139.86 98.785) (end 139.275 98.2) (width 0.5) (layer "F.Cu") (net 14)))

